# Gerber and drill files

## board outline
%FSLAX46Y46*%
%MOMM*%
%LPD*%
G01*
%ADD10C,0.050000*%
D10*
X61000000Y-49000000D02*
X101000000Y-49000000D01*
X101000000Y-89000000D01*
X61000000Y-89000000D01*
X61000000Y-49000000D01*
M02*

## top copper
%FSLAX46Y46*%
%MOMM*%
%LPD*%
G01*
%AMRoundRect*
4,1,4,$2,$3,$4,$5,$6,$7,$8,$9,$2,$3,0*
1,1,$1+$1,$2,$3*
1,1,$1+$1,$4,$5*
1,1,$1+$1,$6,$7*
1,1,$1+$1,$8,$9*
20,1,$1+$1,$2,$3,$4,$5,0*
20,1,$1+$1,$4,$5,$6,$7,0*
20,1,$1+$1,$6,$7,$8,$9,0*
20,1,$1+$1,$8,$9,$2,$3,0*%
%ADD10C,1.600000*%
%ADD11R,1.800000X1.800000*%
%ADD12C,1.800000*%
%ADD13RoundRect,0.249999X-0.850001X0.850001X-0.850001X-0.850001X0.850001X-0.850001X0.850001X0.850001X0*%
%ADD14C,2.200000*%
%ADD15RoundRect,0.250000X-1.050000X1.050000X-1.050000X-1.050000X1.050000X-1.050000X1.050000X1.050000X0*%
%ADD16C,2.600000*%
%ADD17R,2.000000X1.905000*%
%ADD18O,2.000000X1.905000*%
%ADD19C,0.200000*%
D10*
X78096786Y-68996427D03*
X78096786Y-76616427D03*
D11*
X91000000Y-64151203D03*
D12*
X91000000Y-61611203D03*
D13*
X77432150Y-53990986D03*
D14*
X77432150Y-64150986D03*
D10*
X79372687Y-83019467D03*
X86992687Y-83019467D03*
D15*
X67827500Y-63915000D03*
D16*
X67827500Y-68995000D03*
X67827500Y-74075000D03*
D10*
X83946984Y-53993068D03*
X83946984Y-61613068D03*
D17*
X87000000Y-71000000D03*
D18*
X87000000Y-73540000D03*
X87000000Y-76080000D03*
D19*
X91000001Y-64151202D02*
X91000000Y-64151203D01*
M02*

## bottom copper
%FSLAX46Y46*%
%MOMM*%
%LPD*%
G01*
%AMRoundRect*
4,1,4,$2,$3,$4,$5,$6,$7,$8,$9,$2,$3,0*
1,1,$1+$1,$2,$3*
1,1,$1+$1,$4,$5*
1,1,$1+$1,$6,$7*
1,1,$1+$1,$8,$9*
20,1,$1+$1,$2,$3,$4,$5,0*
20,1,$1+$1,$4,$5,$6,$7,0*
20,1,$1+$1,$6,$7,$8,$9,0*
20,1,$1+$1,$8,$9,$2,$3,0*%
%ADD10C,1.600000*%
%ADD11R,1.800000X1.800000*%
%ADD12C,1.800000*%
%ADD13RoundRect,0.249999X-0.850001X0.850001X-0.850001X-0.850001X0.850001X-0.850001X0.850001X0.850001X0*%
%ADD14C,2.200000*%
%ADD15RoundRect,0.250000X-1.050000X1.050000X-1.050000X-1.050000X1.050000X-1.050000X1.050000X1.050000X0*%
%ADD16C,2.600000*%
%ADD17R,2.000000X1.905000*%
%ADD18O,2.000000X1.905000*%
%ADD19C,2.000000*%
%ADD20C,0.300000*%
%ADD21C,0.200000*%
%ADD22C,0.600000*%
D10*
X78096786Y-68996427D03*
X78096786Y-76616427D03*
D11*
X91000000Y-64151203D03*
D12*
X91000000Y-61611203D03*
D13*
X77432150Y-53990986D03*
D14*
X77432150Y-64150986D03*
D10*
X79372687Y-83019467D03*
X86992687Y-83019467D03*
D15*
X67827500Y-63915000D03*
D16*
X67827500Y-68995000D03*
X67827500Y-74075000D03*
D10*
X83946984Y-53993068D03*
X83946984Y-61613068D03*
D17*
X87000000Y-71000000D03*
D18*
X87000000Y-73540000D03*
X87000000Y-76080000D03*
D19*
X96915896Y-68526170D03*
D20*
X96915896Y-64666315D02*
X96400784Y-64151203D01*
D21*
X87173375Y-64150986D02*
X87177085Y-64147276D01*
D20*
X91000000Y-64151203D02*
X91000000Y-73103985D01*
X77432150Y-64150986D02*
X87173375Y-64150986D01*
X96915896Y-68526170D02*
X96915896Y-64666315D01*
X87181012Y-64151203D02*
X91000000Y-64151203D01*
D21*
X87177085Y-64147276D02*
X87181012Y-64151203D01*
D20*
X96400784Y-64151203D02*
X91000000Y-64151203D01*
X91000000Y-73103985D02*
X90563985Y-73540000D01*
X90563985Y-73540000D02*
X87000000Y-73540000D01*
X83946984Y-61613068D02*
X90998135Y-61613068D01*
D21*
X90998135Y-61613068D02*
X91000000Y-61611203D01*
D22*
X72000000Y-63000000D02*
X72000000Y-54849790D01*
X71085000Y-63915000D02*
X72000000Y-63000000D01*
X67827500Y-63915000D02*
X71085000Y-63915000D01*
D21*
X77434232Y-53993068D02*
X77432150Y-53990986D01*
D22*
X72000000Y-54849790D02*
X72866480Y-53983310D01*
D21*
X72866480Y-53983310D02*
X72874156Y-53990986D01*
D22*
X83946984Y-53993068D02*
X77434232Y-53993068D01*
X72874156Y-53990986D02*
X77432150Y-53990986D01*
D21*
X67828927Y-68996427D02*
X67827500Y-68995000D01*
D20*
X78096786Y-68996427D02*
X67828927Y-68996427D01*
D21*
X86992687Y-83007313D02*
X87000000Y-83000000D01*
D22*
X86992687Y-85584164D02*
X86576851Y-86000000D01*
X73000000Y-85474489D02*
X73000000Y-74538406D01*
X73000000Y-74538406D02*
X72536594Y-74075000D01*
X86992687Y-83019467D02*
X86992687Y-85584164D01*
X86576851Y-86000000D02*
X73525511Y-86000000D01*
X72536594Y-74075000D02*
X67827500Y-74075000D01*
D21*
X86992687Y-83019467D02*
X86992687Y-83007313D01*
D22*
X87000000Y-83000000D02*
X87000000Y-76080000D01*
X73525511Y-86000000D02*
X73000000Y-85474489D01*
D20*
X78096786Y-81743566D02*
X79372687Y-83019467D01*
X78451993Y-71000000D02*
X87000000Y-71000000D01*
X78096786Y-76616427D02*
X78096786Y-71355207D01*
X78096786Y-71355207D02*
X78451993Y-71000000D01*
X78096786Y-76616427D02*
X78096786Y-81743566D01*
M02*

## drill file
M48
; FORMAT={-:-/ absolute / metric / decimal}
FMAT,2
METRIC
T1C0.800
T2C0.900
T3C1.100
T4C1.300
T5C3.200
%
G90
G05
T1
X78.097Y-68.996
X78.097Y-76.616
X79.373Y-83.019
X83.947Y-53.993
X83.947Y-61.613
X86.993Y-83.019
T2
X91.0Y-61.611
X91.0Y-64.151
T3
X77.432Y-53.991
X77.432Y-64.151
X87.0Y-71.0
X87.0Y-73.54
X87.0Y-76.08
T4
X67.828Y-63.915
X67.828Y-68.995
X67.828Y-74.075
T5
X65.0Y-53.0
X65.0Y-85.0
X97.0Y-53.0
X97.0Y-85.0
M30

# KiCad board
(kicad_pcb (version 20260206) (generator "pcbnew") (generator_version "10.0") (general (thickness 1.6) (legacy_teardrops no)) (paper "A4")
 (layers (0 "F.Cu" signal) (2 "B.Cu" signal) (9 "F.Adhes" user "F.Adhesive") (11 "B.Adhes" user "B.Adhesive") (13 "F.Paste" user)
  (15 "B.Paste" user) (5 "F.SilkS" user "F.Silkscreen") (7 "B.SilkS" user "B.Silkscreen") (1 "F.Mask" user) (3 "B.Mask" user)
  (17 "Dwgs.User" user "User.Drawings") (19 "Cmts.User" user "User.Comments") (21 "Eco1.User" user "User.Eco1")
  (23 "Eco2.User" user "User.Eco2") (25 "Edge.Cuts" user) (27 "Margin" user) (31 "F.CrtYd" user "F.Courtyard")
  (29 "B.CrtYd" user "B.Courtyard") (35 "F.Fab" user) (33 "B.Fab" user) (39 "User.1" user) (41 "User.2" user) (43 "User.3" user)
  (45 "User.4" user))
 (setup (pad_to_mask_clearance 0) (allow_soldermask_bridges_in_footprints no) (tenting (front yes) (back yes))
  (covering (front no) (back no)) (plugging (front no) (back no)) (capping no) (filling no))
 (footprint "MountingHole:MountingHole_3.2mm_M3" (layer "F.Cu") (at 65 53)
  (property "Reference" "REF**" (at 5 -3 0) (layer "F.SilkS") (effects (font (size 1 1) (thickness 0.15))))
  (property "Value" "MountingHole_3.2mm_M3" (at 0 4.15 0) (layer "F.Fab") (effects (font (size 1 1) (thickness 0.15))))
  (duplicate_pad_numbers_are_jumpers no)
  (pad "" np_thru_hole circle (at 0 0) (size 3.2 3.2) (drill 3.2) (layers "*.Cu" "*.Mask")))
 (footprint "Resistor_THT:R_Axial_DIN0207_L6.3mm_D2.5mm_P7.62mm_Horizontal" (layer "F.Cu") (at 78.096786 68.996427 -90)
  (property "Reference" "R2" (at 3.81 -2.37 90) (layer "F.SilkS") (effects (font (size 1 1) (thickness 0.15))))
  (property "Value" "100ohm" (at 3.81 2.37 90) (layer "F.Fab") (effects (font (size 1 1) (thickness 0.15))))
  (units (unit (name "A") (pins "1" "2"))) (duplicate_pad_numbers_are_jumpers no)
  (pad "1" thru_hole circle (at 0 0 270) (size 1.6 1.6) (drill 0.8) (layers "*.Cu" "*.Mask") (remove_unused_layers no)
   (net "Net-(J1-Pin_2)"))
  (pad "2" thru_hole circle (at 7.62 0 270) (size 1.6 1.6) (drill 0.8) (layers "*.Cu" "*.Mask") (remove_unused_layers no) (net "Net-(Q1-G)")))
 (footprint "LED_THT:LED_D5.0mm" (layer "F.Cu") (at 91 64.151203 90)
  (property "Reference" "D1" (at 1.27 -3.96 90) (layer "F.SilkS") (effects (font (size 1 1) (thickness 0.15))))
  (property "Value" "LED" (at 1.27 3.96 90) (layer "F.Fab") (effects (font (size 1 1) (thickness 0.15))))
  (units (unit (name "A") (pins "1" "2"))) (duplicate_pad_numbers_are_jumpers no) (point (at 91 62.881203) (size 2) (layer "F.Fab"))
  (pad "1" thru_hole rect (at 0 0 90) (size 1.8 1.8) (drill 0.9) (layers "*.Cu" "*.Mask") (remove_unused_layers no) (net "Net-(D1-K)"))
  (pad "2" thru_hole circle (at 2.54 0 90) (size 1.8 1.8) (drill 0.9) (layers "*.Cu" "*.Mask") (remove_unused_layers no) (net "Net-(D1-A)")))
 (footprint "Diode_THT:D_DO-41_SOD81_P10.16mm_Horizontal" (layer "F.Cu") (at 77.43215 53.990986 -90)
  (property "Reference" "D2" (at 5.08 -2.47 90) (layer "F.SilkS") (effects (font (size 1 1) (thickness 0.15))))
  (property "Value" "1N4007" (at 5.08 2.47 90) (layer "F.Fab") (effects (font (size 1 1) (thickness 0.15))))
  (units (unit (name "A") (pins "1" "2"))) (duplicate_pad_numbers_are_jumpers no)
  (pad "1" thru_hole roundrect (at 0 0 270) (size 2.2 2.2) (drill 1.1) (layers "*.Cu" "*.Mask") (remove_unused_layers no)
   (roundrect_rratio 0.113636) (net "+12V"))
  (pad "2" thru_hole circle (at 10.16 0 270) (size 2.2 2.2) (drill 1.1) (layers "*.Cu" "*.Mask") (remove_unused_layers no)
   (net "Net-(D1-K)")))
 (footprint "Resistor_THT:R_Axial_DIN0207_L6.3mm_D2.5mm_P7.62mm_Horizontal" (layer "F.Cu") (at 79.372687 83.019467)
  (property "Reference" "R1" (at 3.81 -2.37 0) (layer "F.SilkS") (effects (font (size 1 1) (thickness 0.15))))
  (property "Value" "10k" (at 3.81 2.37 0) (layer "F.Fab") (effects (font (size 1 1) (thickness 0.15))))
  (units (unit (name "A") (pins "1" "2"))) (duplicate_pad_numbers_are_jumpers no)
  (pad "1" thru_hole circle (at 0 0) (size 1.6 1.6) (drill 0.8) (layers "*.Cu" "*.Mask") (remove_unused_layers no) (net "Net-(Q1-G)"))
  (pad "2" thru_hole circle (at 7.62 0) (size 1.6 1.6) (drill 0.8) (layers "*.Cu" "*.Mask") (remove_unused_layers no) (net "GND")))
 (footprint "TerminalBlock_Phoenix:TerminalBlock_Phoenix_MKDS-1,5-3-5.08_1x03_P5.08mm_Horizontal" (layer "F.Cu") (at 67.8275 63.915 -90)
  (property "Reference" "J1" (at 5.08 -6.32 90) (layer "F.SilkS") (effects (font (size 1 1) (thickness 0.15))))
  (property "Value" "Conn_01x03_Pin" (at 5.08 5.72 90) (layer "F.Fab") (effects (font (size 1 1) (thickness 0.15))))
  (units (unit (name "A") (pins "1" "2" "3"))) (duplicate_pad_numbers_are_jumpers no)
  (pad "1" thru_hole roundrect (at 0 0 270) (size 2.6 2.6) (drill 1.3) (layers "*.Cu" "*.Mask") (remove_unused_layers no)
   (roundrect_rratio 0.096154) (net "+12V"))
  (pad "2" thru_hole circle (at 5.08 0 270) (size 2.6 2.6) (drill 1.3) (layers "*.Cu" "*.Mask") (remove_unused_layers no)
   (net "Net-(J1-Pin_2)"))
  (pad "3" thru_hole circle (at 10.16 0 270) (size 2.6 2.6) (drill 1.3) (layers "*.Cu" "*.Mask") (remove_unused_layers no) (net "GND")))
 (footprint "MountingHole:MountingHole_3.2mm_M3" (layer "F.Cu") (at 97 85)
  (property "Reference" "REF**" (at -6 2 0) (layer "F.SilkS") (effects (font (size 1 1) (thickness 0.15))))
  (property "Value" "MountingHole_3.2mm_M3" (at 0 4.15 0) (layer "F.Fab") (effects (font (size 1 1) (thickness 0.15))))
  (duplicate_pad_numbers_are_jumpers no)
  (pad "" np_thru_hole circle (at 0 0) (size 3.2 3.2) (drill 3.2) (layers "*.Cu" "*.Mask")))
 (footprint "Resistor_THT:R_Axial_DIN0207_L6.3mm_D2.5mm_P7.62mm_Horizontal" (layer "F.Cu") (at 83.946984 53.993068 -90)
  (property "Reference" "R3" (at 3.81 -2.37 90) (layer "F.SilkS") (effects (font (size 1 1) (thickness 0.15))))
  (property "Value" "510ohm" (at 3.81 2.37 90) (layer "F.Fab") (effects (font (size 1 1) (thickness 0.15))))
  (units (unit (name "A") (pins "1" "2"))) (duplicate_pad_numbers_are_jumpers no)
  (pad "1" thru_hole circle (at 0 0 270) (size 1.6 1.6) (drill 0.8) (layers "*.Cu" "*.Mask") (remove_unused_layers no) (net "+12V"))
  (pad "2" thru_hole circle (at 7.62 0 270) (size 1.6 1.6) (drill 0.8) (layers "*.Cu" "*.Mask") (remove_unused_layers no) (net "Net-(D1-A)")))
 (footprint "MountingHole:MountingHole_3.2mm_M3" (layer "F.Cu") (at 97 53)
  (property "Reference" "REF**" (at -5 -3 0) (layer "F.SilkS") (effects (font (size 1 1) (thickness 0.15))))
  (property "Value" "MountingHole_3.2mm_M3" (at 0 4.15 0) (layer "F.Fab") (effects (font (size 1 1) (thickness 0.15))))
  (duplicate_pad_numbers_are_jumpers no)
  (pad "" np_thru_hole circle (at 0 0) (size 3.2 3.2) (drill 3.2) (layers "*.Cu" "*.Mask")))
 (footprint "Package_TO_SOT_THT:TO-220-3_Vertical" (layer "F.Cu") (at 87 71 -90)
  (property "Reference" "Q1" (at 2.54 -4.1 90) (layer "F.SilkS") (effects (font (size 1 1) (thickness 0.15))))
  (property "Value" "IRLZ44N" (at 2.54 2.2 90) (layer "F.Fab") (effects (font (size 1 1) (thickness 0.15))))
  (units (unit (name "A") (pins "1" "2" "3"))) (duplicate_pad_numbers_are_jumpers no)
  (pad "1" thru_hole rect (at 0 0 270) (size 1.905 2) (drill 1.1) (layers "*.Cu" "*.Mask") (remove_unused_layers no) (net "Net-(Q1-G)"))
  (pad "2" thru_hole oval (at 2.54 0 270) (size 1.905 2) (drill 1.1) (layers "*.Cu" "*.Mask") (remove_unused_layers no) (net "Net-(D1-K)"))
  (pad "3" thru_hole oval (at 5.08 0 270) (size 1.905 2) (drill 1.1) (layers "*.Cu" "*.Mask") (remove_unused_layers no) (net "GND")))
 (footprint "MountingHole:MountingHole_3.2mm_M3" (layer "F.Cu") (at 65 85)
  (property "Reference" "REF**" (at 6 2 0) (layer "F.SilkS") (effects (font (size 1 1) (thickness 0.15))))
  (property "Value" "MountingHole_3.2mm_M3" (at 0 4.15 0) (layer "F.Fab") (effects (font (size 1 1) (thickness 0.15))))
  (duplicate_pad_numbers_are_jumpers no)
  (pad "" np_thru_hole circle (at 0 0) (size 3.2 3.2) (drill 3.2) (layers "*.Cu" "*.Mask")))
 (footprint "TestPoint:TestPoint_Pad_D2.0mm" (layer "B.Cu") (at 96.915896 68.52617 180)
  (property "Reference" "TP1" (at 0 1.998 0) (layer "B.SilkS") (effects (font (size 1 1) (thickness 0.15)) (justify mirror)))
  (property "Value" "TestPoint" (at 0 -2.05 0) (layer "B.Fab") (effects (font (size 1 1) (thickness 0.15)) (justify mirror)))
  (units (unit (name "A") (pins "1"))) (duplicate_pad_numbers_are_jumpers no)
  (pad "1" smd circle (at 0 0 180) (size 2 2) (layers "B.Cu" "B.Mask") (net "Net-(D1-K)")))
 (gr_rect (start 61 49) (end 101 89) (stroke (width 0.05) (type default)) (fill no) (layer "Edge.Cuts"))
 (segment (start 91.000001 64.151202) (end 91 64.151203) (width 0.2) (layer "F.Cu") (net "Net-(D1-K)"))
 (segment (start 96.915896 64.666315) (end 96.400784 64.151203) (width 0.3) (layer "B.Cu") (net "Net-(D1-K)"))
 (segment (start 87.173375 64.150986) (end 87.177085 64.147276) (width 0.2) (layer "B.Cu") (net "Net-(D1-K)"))
 (segment (start 91 64.151203) (end 91 73.103985) (width 0.3) (layer "B.Cu") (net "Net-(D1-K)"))
 (segment (start 77.43215 64.150986) (end 87.173375 64.150986) (width 0.3) (layer "B.Cu") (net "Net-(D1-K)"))
 (segment (start 96.915896 68.52617) (end 96.915896 64.666315) (width 0.3) (layer "B.Cu") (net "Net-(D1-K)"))
 (segment (start 87.181012 64.151203) (end 91 64.151203) (width 0.3) (layer "B.Cu") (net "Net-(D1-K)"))
 (segment (start 87.177085 64.147276) (end 87.181012 64.151203) (width 0.2) (layer "B.Cu") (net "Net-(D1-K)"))
 (segment (start 96.400784 64.151203) (end 91 64.151203) (width 0.3) (layer "B.Cu") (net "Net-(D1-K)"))
 (segment (start 91 73.103985) (end 90.563985 73.54) (width 0.3) (layer "B.Cu") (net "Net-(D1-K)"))
 (segment (start 90.563985 73.54) (end 87 73.54) (width 0.3) (layer "B.Cu") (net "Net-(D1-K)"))
 (segment (start 83.946984 61.613068) (end 90.998135 61.613068) (width 0.3) (layer "B.Cu") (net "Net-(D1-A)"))
 (segment (start 90.998135 61.613068) (end 91 61.611203) (width 0.2) (layer "B.Cu") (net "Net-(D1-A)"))
 (segment (start 72 63) (end 72 54.84979) (width 0.6) (layer "B.Cu") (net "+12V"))
 (segment (start 71.085 63.915) (end 72 63) (width 0.6) (layer "B.Cu") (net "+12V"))
 (segment (start 67.8275 63.915) (end 71.085 63.915) (width 0.6) (layer "B.Cu") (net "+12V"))
 (segment (start 77.434232 53.993068) (end 77.43215 53.990986) (width 0.2) (layer "B.Cu") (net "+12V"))
 (segment (start 72 54.84979) (end 72.86648 53.98331) (width 0.6) (layer "B.Cu") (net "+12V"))
 (segment (start 72.86648 53.98331) (end 72.874156 53.990986) (width 0.2) (layer "B.Cu") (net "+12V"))
 (segment (start 83.946984 53.993068) (end 77.434232 53.993068) (width 0.6) (layer "B.Cu") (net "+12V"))
 (segment (start 72.874156 53.990986) (end 77.43215 53.990986) (width 0.6) (layer "B.Cu") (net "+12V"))
 (segment (start 67.828927 68.996427) (end 67.8275 68.995) (width 0.2) (layer "B.Cu") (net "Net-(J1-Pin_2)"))
 (segment (start 78.096786 68.996427) (end 67.828927 68.996427) (width 0.3) (layer "B.Cu") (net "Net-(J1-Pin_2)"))
 (segment (start 86.992687 83.007313) (end 87 83) (width 0.2) (layer "B.Cu") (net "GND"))
 (segment (start 86.992687 85.584164) (end 86.576851 86) (width 0.6) (layer "B.Cu") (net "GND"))
 (segment (start 73 85.474489) (end 73 74.538406) (width 0.6) (layer "B.Cu") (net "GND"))
 (segment (start 73 74.538406) (end 72.536594 74.075) (width 0.6) (layer "B.Cu") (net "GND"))
 (segment (start 86.992687 83.019467) (end 86.992687 85.584164) (width 0.6) (layer "B.Cu") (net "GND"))
 (segment (start 86.576851 86) (end 73.525511 86) (width 0.6) (layer "B.Cu") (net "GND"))
 (segment (start 72.536594 74.075) (end 67.8275 74.075) (width 0.6) (layer "B.Cu") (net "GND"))
 (segment (start 86.992687 83.019467) (end 86.992687 83.007313) (width 0.2) (layer "B.Cu") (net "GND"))
 (segment (start 87 83) (end 87 76.08) (width 0.6) (layer "B.Cu") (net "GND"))
 (segment (start 73.525511 86) (end 73 85.474489) (width 0.6) (layer "B.Cu") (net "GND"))
 (segment (start 78.096786 81.743566) (end 79.372687 83.019467) (width 0.3) (layer "B.Cu") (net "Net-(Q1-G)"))
 (segment (start 78.451993 71) (end 87 71) (width 0.3) (layer "B.Cu") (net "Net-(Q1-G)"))
 (segment (start 78.096786 76.616427) (end 78.096786 71.355207) (width 0.3) (layer "B.Cu") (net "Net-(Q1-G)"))
 (segment (start 78.096786 71.355207) (end 78.451993 71) (width 0.3) (layer "B.Cu") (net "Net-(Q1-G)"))
 (segment (start 78.096786 76.616427) (end 78.096786 81.743566) (width 0.3) (layer "B.Cu") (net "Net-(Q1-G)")))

